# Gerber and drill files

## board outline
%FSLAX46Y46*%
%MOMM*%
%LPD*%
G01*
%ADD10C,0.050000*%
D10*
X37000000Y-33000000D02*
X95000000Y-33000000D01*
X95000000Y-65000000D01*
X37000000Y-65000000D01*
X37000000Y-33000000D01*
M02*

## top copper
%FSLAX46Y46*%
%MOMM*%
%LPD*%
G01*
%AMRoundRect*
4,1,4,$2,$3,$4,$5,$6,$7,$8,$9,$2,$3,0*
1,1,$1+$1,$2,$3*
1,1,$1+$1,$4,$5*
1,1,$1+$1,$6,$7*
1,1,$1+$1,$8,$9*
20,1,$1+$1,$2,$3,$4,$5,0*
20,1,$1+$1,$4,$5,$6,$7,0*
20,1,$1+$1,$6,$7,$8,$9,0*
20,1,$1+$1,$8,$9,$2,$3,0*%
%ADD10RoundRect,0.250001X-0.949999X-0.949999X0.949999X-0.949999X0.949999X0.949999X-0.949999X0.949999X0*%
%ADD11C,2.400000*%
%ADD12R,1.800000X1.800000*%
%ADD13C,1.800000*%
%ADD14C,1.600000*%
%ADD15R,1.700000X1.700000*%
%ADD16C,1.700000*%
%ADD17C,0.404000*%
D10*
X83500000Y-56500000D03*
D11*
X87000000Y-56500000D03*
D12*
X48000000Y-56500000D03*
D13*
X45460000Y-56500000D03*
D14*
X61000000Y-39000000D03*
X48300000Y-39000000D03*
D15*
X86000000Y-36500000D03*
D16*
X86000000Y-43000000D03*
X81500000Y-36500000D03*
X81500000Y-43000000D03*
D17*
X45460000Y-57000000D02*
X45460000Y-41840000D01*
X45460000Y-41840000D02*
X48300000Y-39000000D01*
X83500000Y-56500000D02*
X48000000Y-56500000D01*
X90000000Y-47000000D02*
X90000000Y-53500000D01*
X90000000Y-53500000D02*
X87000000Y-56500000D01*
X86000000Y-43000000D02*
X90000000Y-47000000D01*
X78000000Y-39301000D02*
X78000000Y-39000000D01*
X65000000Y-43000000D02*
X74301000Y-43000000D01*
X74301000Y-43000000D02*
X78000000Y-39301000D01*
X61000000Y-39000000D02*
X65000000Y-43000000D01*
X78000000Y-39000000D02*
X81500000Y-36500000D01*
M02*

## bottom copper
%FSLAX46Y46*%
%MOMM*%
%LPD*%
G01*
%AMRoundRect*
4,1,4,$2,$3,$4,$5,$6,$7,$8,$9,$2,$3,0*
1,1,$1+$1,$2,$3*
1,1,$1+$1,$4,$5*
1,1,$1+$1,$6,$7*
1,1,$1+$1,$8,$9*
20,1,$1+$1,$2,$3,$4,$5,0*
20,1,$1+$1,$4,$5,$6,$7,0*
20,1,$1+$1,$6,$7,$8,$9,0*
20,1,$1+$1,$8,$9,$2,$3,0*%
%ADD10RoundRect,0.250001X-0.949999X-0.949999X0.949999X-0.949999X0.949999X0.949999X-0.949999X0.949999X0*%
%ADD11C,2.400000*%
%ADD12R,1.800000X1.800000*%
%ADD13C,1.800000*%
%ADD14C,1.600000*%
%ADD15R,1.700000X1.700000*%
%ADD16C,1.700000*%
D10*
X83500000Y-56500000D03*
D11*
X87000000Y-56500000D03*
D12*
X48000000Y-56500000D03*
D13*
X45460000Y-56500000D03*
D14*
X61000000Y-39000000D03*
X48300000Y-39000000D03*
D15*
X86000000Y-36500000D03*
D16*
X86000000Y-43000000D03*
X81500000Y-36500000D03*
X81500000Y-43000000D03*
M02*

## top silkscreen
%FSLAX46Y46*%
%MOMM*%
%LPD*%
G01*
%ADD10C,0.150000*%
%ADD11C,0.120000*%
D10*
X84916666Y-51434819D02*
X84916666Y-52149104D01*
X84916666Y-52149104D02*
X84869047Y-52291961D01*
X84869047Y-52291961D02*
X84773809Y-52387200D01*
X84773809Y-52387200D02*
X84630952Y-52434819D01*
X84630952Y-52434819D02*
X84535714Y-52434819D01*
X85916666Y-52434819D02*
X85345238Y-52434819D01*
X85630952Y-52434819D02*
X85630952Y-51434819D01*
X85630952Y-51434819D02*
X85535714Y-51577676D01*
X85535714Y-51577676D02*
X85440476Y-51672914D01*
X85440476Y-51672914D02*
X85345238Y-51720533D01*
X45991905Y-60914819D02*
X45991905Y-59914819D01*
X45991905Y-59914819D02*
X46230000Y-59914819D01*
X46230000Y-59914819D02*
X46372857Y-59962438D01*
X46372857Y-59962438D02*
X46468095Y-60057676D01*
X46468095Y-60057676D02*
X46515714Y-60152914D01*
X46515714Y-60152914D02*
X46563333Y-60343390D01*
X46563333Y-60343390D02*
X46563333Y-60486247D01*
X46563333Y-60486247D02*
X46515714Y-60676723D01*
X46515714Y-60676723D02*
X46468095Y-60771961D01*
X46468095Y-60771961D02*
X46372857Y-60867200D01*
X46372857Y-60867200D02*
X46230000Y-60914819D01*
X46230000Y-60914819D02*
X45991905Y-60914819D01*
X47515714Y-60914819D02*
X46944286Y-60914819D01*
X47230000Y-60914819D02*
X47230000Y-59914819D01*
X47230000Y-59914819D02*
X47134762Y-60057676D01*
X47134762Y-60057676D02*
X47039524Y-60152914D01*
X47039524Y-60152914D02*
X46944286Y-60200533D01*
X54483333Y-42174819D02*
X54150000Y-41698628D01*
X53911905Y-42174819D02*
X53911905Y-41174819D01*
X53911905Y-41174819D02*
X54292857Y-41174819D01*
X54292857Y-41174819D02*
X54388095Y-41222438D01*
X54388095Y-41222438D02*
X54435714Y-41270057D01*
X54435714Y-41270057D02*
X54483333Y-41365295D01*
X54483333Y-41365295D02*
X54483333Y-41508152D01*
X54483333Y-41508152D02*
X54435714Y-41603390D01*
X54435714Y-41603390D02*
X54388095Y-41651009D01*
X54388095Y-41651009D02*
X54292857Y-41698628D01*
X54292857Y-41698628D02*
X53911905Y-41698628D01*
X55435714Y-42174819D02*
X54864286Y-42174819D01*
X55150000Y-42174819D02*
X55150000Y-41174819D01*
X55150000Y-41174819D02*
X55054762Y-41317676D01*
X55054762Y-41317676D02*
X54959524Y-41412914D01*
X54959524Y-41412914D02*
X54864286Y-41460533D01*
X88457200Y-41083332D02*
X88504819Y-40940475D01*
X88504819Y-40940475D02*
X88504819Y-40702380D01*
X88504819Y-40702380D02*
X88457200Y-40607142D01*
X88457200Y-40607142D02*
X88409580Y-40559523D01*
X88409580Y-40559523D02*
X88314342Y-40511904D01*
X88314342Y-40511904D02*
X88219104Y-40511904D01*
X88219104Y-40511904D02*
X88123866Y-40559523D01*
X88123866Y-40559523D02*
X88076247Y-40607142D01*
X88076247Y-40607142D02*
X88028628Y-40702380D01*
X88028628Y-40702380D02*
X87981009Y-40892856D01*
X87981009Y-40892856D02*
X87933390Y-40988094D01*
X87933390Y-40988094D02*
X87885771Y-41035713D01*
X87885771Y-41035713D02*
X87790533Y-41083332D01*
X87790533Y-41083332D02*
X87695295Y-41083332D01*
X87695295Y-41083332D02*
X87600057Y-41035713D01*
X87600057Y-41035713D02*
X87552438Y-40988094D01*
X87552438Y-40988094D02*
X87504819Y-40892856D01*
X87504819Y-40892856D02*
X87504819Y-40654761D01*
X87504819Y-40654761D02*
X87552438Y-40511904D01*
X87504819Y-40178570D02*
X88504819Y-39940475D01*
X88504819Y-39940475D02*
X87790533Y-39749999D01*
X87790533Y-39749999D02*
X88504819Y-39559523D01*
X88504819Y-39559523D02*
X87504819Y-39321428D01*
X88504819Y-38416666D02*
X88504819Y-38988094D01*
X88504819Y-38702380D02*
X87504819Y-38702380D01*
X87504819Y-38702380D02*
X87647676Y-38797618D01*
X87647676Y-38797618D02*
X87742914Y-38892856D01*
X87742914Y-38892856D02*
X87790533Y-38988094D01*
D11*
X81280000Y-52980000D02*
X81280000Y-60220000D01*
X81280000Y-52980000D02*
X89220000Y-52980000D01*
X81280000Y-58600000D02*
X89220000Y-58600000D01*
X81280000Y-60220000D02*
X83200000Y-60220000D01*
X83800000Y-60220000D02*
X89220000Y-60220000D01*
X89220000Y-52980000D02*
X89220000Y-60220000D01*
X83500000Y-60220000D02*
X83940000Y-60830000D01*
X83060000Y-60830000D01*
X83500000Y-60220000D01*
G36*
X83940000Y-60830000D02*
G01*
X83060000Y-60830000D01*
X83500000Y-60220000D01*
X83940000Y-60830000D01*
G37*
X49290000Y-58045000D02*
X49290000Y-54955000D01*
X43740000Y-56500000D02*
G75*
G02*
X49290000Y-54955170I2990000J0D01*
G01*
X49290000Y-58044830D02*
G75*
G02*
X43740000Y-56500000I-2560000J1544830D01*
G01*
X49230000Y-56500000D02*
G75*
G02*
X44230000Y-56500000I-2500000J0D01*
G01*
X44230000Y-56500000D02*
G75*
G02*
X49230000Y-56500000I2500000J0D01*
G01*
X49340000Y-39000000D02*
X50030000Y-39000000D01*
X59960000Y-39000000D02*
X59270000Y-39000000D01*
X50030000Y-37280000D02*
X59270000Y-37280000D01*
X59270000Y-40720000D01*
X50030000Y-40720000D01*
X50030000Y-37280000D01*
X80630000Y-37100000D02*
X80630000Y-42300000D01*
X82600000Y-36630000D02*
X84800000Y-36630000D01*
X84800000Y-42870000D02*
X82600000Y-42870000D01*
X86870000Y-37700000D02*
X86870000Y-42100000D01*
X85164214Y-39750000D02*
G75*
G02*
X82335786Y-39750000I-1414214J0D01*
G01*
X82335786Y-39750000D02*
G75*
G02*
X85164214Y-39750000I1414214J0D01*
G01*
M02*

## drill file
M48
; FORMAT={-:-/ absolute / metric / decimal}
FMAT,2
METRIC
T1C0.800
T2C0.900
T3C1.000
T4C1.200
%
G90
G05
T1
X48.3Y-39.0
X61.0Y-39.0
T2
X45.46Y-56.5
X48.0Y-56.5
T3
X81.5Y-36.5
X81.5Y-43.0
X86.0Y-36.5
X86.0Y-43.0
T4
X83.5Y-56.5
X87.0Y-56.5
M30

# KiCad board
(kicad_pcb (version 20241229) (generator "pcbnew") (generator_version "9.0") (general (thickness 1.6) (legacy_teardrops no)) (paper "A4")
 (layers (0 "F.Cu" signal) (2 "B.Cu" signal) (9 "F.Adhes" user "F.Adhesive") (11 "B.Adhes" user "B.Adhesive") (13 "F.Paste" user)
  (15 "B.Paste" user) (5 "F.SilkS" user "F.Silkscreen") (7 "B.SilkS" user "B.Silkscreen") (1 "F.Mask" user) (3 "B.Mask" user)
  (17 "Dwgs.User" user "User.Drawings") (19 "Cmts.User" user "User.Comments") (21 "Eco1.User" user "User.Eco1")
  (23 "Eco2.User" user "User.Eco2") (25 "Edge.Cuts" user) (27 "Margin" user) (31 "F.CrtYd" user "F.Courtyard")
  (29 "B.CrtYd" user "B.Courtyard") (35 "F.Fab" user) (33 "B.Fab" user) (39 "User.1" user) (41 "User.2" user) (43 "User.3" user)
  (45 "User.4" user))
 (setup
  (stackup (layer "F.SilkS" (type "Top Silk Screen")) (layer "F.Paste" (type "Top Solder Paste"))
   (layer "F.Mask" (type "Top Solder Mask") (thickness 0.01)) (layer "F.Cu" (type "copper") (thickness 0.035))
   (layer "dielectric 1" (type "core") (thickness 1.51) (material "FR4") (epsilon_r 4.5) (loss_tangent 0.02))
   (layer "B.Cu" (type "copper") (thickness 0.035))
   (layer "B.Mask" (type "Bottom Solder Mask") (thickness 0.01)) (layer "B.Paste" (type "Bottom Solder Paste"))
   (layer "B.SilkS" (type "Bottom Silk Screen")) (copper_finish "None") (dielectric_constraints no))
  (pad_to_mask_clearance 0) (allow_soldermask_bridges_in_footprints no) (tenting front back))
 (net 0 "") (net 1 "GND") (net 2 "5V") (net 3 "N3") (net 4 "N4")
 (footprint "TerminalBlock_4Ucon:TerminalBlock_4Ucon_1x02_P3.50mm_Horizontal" (layer "F.Cu") (at 83.5 56.5)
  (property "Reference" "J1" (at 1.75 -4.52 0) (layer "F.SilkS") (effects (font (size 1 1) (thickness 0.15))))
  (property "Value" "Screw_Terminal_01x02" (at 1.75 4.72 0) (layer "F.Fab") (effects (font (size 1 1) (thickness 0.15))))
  (fp_line (start -2.22 -3.52) (end -2.22 3.72) (stroke (width 0.12) (type solid)) (layer "F.SilkS"))
  (fp_line (start -2.22 -3.52) (end 5.72 -3.52) (stroke (width 0.12) (type solid)) (layer "F.SilkS"))
  (fp_line (start -2.22 2.1) (end 5.72 2.1) (stroke (width 0.12) (type solid)) (layer "F.SilkS"))
  (fp_line (start -2.22 3.72) (end -0.3 3.72) (stroke (width 0.12) (type solid)) (layer "F.SilkS"))
  (fp_line (start 0.3 3.72) (end 5.72 3.72) (stroke (width 0.12) (type solid)) (layer "F.SilkS"))
  (fp_line (start 5.72 -3.52) (end 5.72 3.72) (stroke (width 0.12) (type solid)) (layer "F.SilkS"))
  (fp_poly (pts (xy 0 3.72) (xy 0.44 4.33) (xy -0.44 4.33)) (stroke (width 0.12) (type solid)) (fill yes) (layer "F.SilkS"))
  (pad "1" thru_hole roundrect (at 0 0) (size 2.4 2.4) (drill 1.2) (layers "*.Cu" "*.Mask") (remove_unused_layers no)
   (roundrect_rratio 0.104167) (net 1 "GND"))
  (pad "2" thru_hole circle (at 3.5 0) (size 2.4 2.4) (drill 1.2) (layers "*.Cu" "*.Mask") (remove_unused_layers no) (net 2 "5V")))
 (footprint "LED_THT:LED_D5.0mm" (layer "F.Cu") (at 48 56.5 180)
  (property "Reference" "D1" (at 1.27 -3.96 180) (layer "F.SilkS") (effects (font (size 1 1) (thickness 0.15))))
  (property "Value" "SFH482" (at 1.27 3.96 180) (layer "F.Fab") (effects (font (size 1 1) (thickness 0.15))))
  (fp_line (start -1.29 -1.545) (end -1.29 1.545) (stroke (width 0.12) (type solid)) (layer "F.SilkS"))
  (fp_arc (start 4.26 0) (mid 2.071779 2.880495) (end -1.29 1.54483) (stroke (width 0.12) (type solid)) (layer "F.SilkS"))
  (fp_arc (start -1.29 -1.54483) (mid 2.071779 -2.880495) (end 4.26 0) (stroke (width 0.12) (type solid)) (layer "F.SilkS"))
  (fp_circle (center 1.27 0) (end 3.77 0) (stroke (width 0.12) (type solid)) (fill no) (layer "F.SilkS"))
  (pad "1" thru_hole rect (at 0 0 180) (size 1.8 1.8) (drill 0.9) (layers "*.Cu" "*.Mask") (remove_unused_layers no) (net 1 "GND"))
  (pad "2" thru_hole circle (at 2.54 0 180) (size 1.8 1.8) (drill 0.9) (layers "*.Cu" "*.Mask") (remove_unused_layers no) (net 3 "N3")))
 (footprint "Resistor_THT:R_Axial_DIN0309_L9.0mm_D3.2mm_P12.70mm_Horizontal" (layer "F.Cu") (at 61 39 180)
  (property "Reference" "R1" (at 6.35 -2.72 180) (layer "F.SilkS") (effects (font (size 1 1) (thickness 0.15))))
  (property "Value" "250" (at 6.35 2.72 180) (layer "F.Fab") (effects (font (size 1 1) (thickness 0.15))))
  (fp_line (start 11.66 0) (end 10.97 0) (stroke (width 0.12) (type solid)) (layer "F.SilkS"))
  (fp_line (start 1.04 0) (end 1.73 0) (stroke (width 0.12) (type solid)) (layer "F.SilkS"))
  (fp_rect (start 1.73 -1.72) (end 10.97 1.72) (stroke (width 0.12) (type solid)) (fill no) (layer "F.SilkS"))
  (pad "1" thru_hole circle (at 0 0 180) (size 1.6 1.6) (drill 0.8) (layers "*.Cu" "*.Mask") (remove_unused_layers no) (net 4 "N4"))
  (pad "2" thru_hole circle (at 12.7 0 180) (size 1.6 1.6) (drill 0.8) (layers "*.Cu" "*.Mask") (remove_unused_layers no) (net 3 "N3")))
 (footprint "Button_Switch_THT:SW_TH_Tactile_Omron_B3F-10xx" (layer "F.Cu") (at 86 36.5 -90)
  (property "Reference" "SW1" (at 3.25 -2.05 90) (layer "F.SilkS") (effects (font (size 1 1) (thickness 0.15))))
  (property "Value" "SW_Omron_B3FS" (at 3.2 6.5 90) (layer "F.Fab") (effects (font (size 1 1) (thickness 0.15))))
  (fp_line (start 0.6 5.37) (end 5.8 5.37) (stroke (width 0.12) (type solid)) (layer "F.SilkS"))
  (fp_line (start 0.13 3.4) (end 0.13 1.2) (stroke (width 0.12) (type solid)) (layer "F.SilkS"))
  (fp_line (start 6.37 1.2) (end 6.37 3.4) (stroke (width 0.12) (type solid)) (layer "F.SilkS"))
  (fp_line (start 1.2 -0.87) (end 5.6 -0.87) (stroke (width 0.12) (type solid)) (layer "F.SilkS"))
  (fp_circle (center 3.25 2.25) (end 4.25 3.25) (stroke (width 0.12) (type solid)) (fill no) (layer "F.SilkS"))
  (pad "1" thru_hole rect (at 0 0 270) (size 1.7 1.7) (drill 1) (layers "*.Cu" "*.Mask") (remove_unused_layers no) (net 2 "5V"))
  (pad "1" thru_hole circle (at 6.5 0 270) (size 1.7 1.7) (drill 1) (layers "*.Cu" "*.Mask") (remove_unused_layers no) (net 2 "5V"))
  (pad "2" thru_hole circle (at 0 4.5 270) (size 1.7 1.7) (drill 1) (layers "*.Cu" "*.Mask") (remove_unused_layers no) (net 4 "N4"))
  (pad "2" thru_hole circle (at 6.5 4.5 270) (size 1.7 1.7) (drill 1) (layers "*.Cu" "*.Mask") (remove_unused_layers no) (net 4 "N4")))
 (gr_rect (start 37 33) (end 95 65) (stroke (width 0.05) (type default)) (fill no) (layer "Edge.Cuts"))
 (segment (start 45.46 57) (end 45.46 41.84) (width 0.404) (layer "F.Cu") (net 3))
 (segment (start 45.46 41.84) (end 48.3 39) (width 0.404) (layer "F.Cu") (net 3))
 (segment (start 83.5 56.5) (end 48 56.5) (width 0.404) (layer "F.Cu") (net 1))
 (segment (start 90 47) (end 90 53.5) (width 0.404) (layer "F.Cu") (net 2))
 (segment (start 90 53.5) (end 87 56.5) (width 0.404) (layer "F.Cu") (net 2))
 (segment (start 86 43) (end 90 47) (width 0.404) (layer "F.Cu") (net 2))
 (segment (start 78 39.301) (end 78 39) (width 0.404) (layer "F.Cu") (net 4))
 (segment (start 65 43) (end 74.301 43) (width 0.404) (layer "F.Cu") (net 4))
 (segment (start 74.301 43) (end 78 39.301) (width 0.404) (layer "F.Cu") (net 4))
 (segment (start 61 39) (end 65 43) (width 0.404) (layer "F.Cu") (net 4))
 (segment (start 78 39) (end 81.5 36.5) (width 0.404) (layer "F.Cu") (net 4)))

